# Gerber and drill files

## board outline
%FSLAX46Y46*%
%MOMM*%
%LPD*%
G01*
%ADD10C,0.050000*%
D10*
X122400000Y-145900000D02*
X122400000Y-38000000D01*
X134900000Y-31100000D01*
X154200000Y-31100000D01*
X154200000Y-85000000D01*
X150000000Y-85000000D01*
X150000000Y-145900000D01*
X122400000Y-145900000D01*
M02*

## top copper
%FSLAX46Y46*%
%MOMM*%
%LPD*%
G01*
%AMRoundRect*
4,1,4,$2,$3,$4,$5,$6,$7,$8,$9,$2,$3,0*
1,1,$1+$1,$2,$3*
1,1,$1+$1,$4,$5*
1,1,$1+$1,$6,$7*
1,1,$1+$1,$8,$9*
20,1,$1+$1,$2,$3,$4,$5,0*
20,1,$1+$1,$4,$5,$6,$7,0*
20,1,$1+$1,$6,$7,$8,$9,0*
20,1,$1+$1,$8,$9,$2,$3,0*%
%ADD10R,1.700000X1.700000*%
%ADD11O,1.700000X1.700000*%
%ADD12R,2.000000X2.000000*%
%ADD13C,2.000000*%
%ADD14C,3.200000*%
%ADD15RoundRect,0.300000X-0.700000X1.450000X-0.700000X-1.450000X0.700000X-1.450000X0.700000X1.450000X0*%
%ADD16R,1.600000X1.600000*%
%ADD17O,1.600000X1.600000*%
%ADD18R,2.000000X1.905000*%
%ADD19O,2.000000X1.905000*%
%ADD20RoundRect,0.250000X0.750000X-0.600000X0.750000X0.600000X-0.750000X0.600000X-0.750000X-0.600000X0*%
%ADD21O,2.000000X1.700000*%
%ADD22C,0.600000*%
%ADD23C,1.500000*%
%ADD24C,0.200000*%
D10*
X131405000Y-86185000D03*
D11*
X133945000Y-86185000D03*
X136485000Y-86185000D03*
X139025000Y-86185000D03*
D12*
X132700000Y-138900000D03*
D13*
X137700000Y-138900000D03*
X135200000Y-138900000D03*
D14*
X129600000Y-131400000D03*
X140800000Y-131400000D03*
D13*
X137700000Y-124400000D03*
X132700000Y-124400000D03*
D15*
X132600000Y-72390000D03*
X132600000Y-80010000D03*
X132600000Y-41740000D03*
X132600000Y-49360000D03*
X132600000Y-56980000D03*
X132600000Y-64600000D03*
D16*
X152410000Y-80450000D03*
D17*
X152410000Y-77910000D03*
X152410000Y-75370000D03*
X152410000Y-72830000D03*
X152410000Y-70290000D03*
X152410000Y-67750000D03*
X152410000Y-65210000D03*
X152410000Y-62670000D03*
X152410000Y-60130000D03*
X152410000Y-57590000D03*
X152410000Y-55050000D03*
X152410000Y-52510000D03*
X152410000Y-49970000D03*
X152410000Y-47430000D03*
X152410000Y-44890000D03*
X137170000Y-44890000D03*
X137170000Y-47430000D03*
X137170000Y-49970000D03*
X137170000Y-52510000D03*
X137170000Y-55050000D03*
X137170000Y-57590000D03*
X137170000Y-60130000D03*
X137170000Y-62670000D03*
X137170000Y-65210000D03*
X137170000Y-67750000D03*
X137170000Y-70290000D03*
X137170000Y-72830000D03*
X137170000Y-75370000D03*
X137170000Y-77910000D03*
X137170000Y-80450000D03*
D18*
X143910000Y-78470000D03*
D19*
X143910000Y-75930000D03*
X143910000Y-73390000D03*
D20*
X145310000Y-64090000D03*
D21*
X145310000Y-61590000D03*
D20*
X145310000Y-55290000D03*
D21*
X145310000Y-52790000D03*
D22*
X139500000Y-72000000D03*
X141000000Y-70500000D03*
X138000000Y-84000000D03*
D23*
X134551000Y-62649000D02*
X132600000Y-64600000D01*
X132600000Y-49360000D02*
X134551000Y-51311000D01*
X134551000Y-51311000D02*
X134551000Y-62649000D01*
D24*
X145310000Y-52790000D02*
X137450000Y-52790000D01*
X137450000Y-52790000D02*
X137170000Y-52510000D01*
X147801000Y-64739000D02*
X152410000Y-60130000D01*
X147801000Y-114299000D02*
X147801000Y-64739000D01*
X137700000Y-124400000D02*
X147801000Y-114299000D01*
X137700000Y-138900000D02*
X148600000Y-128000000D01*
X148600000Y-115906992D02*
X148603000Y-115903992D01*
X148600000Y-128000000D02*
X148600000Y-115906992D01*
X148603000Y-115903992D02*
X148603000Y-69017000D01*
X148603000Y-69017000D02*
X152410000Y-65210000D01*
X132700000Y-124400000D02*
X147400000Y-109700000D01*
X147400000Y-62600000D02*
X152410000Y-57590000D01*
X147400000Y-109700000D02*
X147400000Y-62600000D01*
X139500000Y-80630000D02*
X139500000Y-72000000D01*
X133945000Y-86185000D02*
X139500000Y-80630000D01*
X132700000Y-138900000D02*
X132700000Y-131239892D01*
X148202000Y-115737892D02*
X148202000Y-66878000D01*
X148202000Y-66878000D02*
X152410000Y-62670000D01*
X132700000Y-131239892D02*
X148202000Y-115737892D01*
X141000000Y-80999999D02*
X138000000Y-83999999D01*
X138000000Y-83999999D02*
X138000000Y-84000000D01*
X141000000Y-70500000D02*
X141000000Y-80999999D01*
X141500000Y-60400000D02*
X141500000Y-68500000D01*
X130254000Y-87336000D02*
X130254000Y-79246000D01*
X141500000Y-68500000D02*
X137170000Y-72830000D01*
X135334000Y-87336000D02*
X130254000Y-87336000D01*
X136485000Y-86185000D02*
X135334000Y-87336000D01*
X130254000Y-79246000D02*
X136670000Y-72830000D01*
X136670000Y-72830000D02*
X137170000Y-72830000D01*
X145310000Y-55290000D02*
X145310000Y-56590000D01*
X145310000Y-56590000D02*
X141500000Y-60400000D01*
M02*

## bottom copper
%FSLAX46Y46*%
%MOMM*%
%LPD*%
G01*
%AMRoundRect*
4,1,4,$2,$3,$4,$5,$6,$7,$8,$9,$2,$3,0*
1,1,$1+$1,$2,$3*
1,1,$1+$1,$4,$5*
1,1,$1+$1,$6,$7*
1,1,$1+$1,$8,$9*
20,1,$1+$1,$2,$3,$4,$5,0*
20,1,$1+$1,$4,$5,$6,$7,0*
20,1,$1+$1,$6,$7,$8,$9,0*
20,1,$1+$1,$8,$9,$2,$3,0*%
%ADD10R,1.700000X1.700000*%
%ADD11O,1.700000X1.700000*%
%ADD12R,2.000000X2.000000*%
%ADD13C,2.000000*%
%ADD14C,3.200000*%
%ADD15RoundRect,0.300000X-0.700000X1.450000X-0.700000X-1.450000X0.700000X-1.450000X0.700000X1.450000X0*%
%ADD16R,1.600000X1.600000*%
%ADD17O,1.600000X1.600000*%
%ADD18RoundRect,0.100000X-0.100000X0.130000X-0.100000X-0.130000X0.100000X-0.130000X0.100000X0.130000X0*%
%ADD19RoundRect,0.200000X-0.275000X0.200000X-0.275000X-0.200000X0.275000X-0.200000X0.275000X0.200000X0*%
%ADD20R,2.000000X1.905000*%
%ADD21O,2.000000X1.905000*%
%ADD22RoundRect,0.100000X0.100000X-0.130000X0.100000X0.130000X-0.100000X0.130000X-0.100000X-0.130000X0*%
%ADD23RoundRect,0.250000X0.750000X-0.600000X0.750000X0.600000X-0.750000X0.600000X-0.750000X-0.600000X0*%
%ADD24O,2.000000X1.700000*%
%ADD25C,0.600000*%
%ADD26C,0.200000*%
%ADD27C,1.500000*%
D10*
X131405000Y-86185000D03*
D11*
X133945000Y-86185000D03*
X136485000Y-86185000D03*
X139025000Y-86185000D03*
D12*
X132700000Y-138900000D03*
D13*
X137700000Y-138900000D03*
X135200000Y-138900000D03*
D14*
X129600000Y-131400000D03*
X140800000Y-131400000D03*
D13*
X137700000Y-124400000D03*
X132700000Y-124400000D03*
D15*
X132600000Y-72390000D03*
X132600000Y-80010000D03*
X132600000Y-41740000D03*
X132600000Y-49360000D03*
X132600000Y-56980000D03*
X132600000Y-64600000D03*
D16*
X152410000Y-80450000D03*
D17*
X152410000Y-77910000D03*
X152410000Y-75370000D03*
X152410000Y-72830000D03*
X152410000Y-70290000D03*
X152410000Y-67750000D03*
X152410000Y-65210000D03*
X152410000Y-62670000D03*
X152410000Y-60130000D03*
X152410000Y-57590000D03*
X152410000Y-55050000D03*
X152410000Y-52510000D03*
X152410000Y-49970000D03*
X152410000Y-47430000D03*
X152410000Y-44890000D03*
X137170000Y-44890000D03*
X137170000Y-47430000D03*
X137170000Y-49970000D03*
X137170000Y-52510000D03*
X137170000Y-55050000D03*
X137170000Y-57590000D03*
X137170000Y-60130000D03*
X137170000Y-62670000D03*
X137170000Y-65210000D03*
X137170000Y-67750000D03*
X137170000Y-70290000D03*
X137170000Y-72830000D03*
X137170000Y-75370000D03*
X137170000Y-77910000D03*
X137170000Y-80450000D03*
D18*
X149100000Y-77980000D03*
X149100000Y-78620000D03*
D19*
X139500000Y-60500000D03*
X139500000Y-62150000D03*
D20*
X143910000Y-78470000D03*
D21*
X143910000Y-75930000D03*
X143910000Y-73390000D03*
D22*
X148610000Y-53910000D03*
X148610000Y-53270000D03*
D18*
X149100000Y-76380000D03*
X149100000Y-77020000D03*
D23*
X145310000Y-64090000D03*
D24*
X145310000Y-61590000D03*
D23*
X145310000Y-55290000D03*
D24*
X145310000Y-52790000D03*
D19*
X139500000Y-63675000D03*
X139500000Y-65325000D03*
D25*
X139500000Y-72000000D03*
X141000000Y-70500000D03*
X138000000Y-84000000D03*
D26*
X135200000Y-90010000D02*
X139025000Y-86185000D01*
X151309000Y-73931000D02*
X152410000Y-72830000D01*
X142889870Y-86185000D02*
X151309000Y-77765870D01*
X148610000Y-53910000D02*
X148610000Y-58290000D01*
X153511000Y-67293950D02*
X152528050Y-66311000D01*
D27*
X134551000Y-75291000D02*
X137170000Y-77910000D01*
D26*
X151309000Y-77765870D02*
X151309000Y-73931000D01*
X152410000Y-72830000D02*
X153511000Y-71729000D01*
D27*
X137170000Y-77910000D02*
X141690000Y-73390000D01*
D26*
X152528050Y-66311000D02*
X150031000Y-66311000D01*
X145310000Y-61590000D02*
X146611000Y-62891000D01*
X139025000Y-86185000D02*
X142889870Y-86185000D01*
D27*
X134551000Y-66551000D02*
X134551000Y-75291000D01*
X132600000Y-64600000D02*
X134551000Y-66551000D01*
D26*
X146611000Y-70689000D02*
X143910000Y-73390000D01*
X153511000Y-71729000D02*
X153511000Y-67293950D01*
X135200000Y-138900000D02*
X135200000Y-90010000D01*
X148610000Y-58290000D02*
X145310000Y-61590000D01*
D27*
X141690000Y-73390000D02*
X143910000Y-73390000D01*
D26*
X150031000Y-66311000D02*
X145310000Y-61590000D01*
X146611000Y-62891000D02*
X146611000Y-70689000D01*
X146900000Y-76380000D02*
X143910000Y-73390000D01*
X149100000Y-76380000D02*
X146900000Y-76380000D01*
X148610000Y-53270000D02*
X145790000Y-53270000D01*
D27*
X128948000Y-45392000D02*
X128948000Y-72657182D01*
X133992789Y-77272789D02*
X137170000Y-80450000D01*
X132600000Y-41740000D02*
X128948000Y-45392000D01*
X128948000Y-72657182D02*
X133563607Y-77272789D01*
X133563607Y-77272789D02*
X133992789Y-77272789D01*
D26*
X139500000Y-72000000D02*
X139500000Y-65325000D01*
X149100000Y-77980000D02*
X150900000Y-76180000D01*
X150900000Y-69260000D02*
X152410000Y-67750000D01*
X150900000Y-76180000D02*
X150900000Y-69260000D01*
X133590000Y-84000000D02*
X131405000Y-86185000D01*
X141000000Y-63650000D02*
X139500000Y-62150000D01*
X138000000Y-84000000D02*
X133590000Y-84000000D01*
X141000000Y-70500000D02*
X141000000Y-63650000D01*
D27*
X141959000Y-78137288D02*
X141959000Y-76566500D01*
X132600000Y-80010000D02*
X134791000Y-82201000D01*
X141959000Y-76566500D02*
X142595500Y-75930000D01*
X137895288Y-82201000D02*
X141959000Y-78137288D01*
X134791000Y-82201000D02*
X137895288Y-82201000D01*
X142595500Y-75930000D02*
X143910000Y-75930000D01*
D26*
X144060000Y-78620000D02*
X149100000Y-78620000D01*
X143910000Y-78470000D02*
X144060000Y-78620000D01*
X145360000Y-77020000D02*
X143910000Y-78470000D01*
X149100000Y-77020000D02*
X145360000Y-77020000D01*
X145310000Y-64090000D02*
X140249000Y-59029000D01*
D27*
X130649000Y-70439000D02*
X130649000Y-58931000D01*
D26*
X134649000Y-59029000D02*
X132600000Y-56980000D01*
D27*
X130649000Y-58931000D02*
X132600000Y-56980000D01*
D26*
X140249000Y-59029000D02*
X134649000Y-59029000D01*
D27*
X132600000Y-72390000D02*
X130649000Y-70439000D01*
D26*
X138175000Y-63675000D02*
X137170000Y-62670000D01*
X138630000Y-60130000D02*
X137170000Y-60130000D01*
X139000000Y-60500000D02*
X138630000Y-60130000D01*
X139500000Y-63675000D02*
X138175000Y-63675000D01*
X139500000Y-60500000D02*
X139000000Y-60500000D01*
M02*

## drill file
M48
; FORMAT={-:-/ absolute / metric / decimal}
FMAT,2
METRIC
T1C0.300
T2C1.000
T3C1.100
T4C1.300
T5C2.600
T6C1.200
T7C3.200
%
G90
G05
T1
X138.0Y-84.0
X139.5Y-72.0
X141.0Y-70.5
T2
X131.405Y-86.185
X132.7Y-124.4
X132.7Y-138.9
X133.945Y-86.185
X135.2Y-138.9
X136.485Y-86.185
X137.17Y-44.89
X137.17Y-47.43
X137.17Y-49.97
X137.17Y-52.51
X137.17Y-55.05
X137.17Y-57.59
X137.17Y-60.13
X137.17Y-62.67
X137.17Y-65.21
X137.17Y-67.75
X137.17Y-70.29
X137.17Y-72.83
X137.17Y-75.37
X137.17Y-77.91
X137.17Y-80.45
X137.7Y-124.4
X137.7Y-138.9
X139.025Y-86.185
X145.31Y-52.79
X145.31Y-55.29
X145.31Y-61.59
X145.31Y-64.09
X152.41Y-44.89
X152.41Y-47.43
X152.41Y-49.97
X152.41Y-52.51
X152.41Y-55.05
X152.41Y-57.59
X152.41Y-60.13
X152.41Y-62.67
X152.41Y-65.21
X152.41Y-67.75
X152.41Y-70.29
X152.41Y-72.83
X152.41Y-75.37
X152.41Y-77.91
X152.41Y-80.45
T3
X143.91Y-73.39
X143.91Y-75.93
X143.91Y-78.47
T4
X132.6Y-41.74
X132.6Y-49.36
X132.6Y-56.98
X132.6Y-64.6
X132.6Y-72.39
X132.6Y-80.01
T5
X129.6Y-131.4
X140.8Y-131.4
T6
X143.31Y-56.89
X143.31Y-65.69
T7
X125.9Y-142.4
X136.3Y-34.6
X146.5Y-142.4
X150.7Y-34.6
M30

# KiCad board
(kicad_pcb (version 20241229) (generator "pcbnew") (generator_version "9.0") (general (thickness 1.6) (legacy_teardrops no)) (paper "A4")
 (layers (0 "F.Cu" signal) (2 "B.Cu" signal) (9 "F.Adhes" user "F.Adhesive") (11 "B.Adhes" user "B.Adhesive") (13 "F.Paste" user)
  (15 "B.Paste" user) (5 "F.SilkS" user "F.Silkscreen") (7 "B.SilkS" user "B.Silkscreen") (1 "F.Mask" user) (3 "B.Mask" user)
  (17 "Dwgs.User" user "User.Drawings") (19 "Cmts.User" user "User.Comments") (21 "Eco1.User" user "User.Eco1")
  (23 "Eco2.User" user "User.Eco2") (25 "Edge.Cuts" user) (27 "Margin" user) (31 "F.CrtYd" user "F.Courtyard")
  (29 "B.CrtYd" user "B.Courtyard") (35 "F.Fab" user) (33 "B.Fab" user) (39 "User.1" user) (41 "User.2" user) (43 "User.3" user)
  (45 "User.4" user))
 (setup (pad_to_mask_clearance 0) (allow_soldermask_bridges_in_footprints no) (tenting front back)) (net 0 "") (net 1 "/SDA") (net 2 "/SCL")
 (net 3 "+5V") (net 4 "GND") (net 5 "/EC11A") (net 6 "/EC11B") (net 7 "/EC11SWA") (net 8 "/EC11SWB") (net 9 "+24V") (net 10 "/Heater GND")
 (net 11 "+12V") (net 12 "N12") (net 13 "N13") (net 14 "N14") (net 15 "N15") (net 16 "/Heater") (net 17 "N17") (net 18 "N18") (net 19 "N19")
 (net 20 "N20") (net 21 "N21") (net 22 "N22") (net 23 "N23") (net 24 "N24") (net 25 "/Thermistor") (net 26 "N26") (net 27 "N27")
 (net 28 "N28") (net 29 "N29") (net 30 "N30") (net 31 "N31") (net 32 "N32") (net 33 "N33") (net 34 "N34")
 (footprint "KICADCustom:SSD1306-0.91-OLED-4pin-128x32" (layer "F.Cu") (at 129.215 122.685 90)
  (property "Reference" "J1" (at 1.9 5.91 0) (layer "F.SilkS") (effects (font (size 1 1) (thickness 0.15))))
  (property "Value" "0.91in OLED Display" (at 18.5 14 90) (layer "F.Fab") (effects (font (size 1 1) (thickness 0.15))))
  (pad "1" thru_hole rect (at 36.5 2.19 90) (size 1.7 1.7) (drill 1) (layers "*.Cu" "*.Mask") (remove_unused_layers no) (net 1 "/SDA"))
  (pad "2" thru_hole oval (at 36.5 4.73 90) (size 1.7 1.7) (drill 1) (layers "*.Cu" "*.Mask") (remove_unused_layers no) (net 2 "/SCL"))
  (pad "3" thru_hole oval (at 36.5 7.27 90) (size 1.7 1.7) (drill 1) (layers "*.Cu" "*.Mask") (remove_unused_layers no) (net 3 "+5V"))
  (pad "4" thru_hole oval (at 36.5 9.81 90) (size 1.7 1.7) (drill 1) (layers "*.Cu" "*.Mask") (remove_unused_layers no) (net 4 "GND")))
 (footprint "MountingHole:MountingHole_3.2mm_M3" (layer "F.Cu") (at 146.5 142.4)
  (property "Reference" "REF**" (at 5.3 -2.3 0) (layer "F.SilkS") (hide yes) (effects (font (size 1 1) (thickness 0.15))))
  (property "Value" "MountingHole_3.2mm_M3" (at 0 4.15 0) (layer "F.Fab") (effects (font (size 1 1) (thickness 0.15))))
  (pad "" np_thru_hole circle (at 0 0) (size 3.2 3.2) (drill 3.2) (layers "*.Cu" "*.Mask")))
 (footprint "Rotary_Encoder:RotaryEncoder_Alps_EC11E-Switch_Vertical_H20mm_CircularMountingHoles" (layer "F.Cu") (at 132.7 138.9 90)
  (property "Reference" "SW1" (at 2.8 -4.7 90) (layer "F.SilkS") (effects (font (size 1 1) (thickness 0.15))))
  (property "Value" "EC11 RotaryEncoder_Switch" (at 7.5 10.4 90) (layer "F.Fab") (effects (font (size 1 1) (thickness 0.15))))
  (pad "A" thru_hole rect (at 0 0 90) (size 2 2) (drill 1) (layers "*.Cu" "*.Mask") (remove_unused_layers no) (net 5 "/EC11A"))
  (pad "B" thru_hole circle (at 0 5 90) (size 2 2) (drill 1) (layers "*.Cu" "*.Mask") (remove_unused_layers no) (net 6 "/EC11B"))
  (pad "C" thru_hole circle (at 0 2.5 90) (size 2 2) (drill 1) (layers "*.Cu" "*.Mask") (remove_unused_layers no) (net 4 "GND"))
  (pad "MP" thru_hole circle (at 7.5 -3.1 90) (size 3.2 3.2) (drill 2.6) (layers "*.Cu" "*.Mask") (remove_unused_layers no))
  (pad "MP" thru_hole circle (at 7.5 8.1 90) (size 3.2 3.2) (drill 2.6) (layers "*.Cu" "*.Mask") (remove_unused_layers no))
  (pad "S1" thru_hole circle (at 14.5 5 90) (size 2 2) (drill 1) (layers "*.Cu" "*.Mask") (remove_unused_layers no) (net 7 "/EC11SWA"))
  (pad "S2" thru_hole circle (at 14.5 0 90) (size 2 2) (drill 1) (layers "*.Cu" "*.Mask") (remove_unused_layers no) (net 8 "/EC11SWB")))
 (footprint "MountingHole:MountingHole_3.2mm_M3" (layer "F.Cu") (at 136.3 34.6)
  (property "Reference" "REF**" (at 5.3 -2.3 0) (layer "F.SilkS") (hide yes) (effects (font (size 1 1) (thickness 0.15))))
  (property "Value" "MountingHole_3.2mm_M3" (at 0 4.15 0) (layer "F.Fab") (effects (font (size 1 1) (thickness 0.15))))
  (pad "" np_thru_hole circle (at 0 0) (size 3.2 3.2) (drill 3.2) (layers "*.Cu" "*.Mask")))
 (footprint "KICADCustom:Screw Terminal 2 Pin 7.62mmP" (layer "F.Cu") (at 132.6 72.39 -90)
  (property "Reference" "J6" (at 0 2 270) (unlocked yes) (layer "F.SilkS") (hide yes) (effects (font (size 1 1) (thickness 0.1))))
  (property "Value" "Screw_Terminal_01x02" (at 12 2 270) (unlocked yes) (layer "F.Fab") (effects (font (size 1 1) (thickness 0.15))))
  (pad "1" thru_hole roundrect (at 0 0 270) (size 3.5 2) (drill 1.3) (layers "*.Cu" "*.Mask") (remove_unused_layers no)
   (roundrect_rratio 0.15) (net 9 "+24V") (thermal_bridge_angle 45))
  (pad "2" thru_hole roundrect (at 7.62 0 270) (size 3.5 2) (drill 1.3) (layers "*.Cu" "*.Mask") (remove_unused_layers no)
   (roundrect_rratio 0.15) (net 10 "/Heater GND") (thermal_bridge_angle 45)))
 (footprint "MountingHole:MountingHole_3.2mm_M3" (layer "F.Cu") (at 150.7 34.6)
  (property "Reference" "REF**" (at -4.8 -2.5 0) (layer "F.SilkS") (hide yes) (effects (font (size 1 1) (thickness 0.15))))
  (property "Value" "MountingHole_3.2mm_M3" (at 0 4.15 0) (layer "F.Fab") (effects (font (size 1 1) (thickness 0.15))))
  (pad "" np_thru_hole circle (at 0 0) (size 3.2 3.2) (drill 3.2) (layers "*.Cu" "*.Mask")))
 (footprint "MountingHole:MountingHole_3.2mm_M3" (layer "F.Cu") (at 125.9 142.4)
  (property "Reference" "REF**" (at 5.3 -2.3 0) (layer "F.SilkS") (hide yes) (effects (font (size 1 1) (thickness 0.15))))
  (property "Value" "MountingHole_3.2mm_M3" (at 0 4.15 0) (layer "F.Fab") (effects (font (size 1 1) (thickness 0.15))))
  (pad "" np_thru_hole circle (at 0 0) (size 3.2 3.2) (drill 3.2) (layers "*.Cu" "*.Mask")))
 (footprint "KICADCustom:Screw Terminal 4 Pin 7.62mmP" (layer "F.Cu") (at 132.6 41.74 -90)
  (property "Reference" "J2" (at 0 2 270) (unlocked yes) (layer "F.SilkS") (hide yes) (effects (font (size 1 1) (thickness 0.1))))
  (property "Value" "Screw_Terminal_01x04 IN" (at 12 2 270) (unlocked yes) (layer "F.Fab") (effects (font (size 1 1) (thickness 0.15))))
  (pad "1" thru_hole roundrect (at 0 0 270) (size 3.5 2) (drill 1.3) (layers "*.Cu" "*.Mask") (remove_unused_layers no)
   (roundrect_rratio 0.15) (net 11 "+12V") (thermal_bridge_angle 45))
  (pad "2" thru_hole roundrect (at 7.62 0 270) (size 3.5 2) (drill 1.3) (layers "*.Cu" "*.Mask") (remove_unused_layers no)
   (roundrect_rratio 0.15) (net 4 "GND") (thermal_bridge_angle 45))
  (pad "3" thru_hole roundrect (at 15.24 0 270) (size 3.5 2) (drill 1.3) (layers "*.Cu" "*.Mask") (remove_unused_layers no)
   (roundrect_rratio 0.15) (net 9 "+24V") (thermal_bridge_angle 45))
  (pad "4" thru_hole roundrect (at 22.86 0 270) (size 3.5 2) (drill 1.3) (layers "*.Cu" "*.Mask") (remove_unused_layers no)
   (roundrect_rratio 0.15) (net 4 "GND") (thermal_bridge_angle 45)))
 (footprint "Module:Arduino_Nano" (layer "F.Cu") (at 152.41 80.45 180)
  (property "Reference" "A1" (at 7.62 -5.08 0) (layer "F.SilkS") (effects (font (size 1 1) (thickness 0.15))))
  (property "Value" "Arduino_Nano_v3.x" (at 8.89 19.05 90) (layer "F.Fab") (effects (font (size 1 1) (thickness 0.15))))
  (pad "1" thru_hole rect (at 0 0 180) (size 1.6 1.6) (drill 1) (layers "*.Cu" "*.Mask") (remove_unused_layers no) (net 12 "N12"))
  (pad "2" thru_hole oval (at 0 2.54 180) (size 1.6 1.6) (drill 1) (layers "*.Cu" "*.Mask") (remove_unused_layers no) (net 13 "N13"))
  (pad "3" thru_hole oval (at 0 5.08 180) (size 1.6 1.6) (drill 1) (layers "*.Cu" "*.Mask") (remove_unused_layers no) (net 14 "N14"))
  (pad "4" thru_hole oval (at 0 7.62 180) (size 1.6 1.6) (drill 1) (layers "*.Cu" "*.Mask") (remove_unused_layers no) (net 4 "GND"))
  (pad "5" thru_hole oval (at 0 10.16 180) (size 1.6 1.6) (drill 1) (layers "*.Cu" "*.Mask") (remove_unused_layers no) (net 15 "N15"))
  (pad "6" thru_hole oval (at 0 12.7 180) (size 1.6 1.6) (drill 1) (layers "*.Cu" "*.Mask") (remove_unused_layers no) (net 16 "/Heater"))
  (pad "7" thru_hole oval (at 0 15.24 180) (size 1.6 1.6) (drill 1) (layers "*.Cu" "*.Mask") (remove_unused_layers no) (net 6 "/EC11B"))
  (pad "8" thru_hole oval (at 0 17.78 180) (size 1.6 1.6) (drill 1) (layers "*.Cu" "*.Mask") (remove_unused_layers no) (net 5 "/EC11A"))
  (pad "9" thru_hole oval (at 0 20.32 180) (size 1.6 1.6) (drill 1) (layers "*.Cu" "*.Mask") (remove_unused_layers no) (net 7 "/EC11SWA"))
  (pad "10" thru_hole oval (at 0 22.86 180) (size 1.6 1.6) (drill 1) (layers "*.Cu" "*.Mask") (remove_unused_layers no) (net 8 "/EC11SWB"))
  (pad "11" thru_hole oval (at 0 25.4 180) (size 1.6 1.6) (drill 1) (layers "*.Cu" "*.Mask") (remove_unused_layers no) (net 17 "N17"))
  (pad "12" thru_hole oval (at 0 27.94 180) (size 1.6 1.6) (drill 1) (layers "*.Cu" "*.Mask") (remove_unused_layers no) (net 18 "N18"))
  (pad "13" thru_hole oval (at 0 30.48 180) (size 1.6 1.6) (drill 1) (layers "*.Cu" "*.Mask") (remove_unused_layers no) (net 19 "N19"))
  (pad "14" thru_hole oval (at 0 33.02 180) (size 1.6 1.6) (drill 1) (layers "*.Cu" "*.Mask") (remove_unused_layers no) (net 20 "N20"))
  (pad "15" thru_hole oval (at 0 35.56 180) (size 1.6 1.6) (drill 1) (layers "*.Cu" "*.Mask") (remove_unused_layers no) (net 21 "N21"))
  (pad "16" thru_hole oval (at 15.24 35.56 180) (size 1.6 1.6) (drill 1) (layers "*.Cu" "*.Mask") (remove_unused_layers no) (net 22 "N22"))
  (pad "17" thru_hole oval (at 15.24 33.02 180) (size 1.6 1.6) (drill 1) (layers "*.Cu" "*.Mask") (remove_unused_layers no) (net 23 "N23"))
  (pad "18" thru_hole oval (at 15.24 30.48 180) (size 1.6 1.6) (drill 1) (layers "*.Cu" "*.Mask") (remove_unused_layers no) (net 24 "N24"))
  (pad "19" thru_hole oval (at 15.24 27.94 180) (size 1.6 1.6) (drill 1) (layers "*.Cu" "*.Mask") (remove_unused_layers no)
   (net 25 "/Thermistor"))
  (pad "20" thru_hole oval (at 15.24 25.4 180) (size 1.6 1.6) (drill 1) (layers "*.Cu" "*.Mask") (remove_unused_layers no) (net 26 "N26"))
  (pad "21" thru_hole oval (at 15.24 22.86 180) (size 1.6 1.6) (drill 1) (layers "*.Cu" "*.Mask") (remove_unused_layers no) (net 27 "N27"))
  (pad "22" thru_hole oval (at 15.24 20.32 180) (size 1.6 1.6) (drill 1) (layers "*.Cu" "*.Mask") (remove_unused_layers no) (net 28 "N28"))
  (pad "23" thru_hole oval (at 15.24 17.78 180) (size 1.6 1.6) (drill 1) (layers "*.Cu" "*.Mask") (remove_unused_layers no) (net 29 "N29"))
  (pad "24" thru_hole oval (at 15.24 15.24 180) (size 1.6 1.6) (drill 1) (layers "*.Cu" "*.Mask") (remove_unused_layers no) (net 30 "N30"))
  (pad "25" thru_hole oval (at 15.24 12.7 180) (size 1.6 1.6) (drill 1) (layers "*.Cu" "*.Mask") (remove_unused_layers no) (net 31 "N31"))
  (pad "26" thru_hole oval (at 15.24 10.16 180) (size 1.6 1.6) (drill 1) (layers "*.Cu" "*.Mask") (remove_unused_layers no) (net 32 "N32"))
  (pad "27" thru_hole oval (at 15.24 7.62 180) (size 1.6 1.6) (drill 1) (layers "*.Cu" "*.Mask") (remove_unused_layers no) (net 3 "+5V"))
  (pad "28" thru_hole oval (at 15.24 5.08 180) (size 1.6 1.6) (drill 1) (layers "*.Cu" "*.Mask") (remove_unused_layers no) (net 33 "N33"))
  (pad "29" thru_hole oval (at 15.24 2.54 180) (size 1.6 1.6) (drill 1) (layers "*.Cu" "*.Mask") (remove_unused_layers no) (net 4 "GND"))
  (pad "30" thru_hole oval (at 15.24 0 180) (size 1.6 1.6) (drill 1) (layers "*.Cu" "*.Mask") (remove_unused_layers no) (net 11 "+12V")))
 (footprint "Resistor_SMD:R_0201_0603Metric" (layer "B.Cu") (at 149.1 78.3 -90)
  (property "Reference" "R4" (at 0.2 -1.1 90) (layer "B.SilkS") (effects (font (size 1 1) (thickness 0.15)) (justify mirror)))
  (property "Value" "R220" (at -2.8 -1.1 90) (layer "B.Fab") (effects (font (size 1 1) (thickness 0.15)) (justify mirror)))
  (pad "" smd roundrect (at -0.345 0 270) (size 0.318 0.36) (layers "B.Paste") (roundrect_rratio 0.25))
  (pad "" smd roundrect (at 0.345 0 270) (size 0.318 0.36) (layers "B.Paste") (roundrect_rratio 0.25))
  (pad "1" smd roundrect (at -0.32 0 270) (size 0.46 0.4) (layers "B.Cu" "B.Mask") (roundrect_rratio 0.25) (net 16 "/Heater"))
  (pad "2" smd roundrect (at 0.32 0 270) (size 0.46 0.4) (layers "B.Cu" "B.Mask") (roundrect_rratio 0.25) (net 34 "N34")))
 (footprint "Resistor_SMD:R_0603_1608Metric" (layer "B.Cu") (at 139.5 61.325 -90)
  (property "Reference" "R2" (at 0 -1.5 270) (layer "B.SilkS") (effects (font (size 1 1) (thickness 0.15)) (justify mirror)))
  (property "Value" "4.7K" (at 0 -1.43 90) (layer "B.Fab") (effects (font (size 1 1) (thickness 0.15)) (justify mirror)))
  (pad "1" smd roundrect (at -0.825 0 270) (size 0.8 0.95) (layers "B.Cu" "B.Mask" "B.Paste") (roundrect_rratio 0.25) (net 29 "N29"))
  (pad "2" smd roundrect (at 0.825 0 270) (size 0.8 0.95) (layers "B.Cu" "B.Mask" "B.Paste") (roundrect_rratio 0.25) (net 1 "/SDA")))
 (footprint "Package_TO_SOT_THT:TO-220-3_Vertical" (layer "B.Cu") (at 143.91 78.47 90)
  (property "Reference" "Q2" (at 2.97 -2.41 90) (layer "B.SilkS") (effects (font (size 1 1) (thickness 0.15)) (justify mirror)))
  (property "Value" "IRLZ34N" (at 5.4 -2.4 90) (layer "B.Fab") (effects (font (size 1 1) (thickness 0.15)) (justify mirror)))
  (pad "1" thru_hole rect (at 0 0 90) (size 1.905 2) (drill 1.1) (layers "*.Cu" "*.Mask") (remove_unused_layers no) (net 34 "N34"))
  (pad "2" thru_hole oval (at 2.54 0 90) (size 1.905 2) (drill 1.1) (layers "*.Cu" "*.Mask") (remove_unused_layers no)
   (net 10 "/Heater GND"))
  (pad "3" thru_hole oval (at 5.08 0 90) (size 1.905 2) (drill 1.1) (layers "*.Cu" "*.Mask") (remove_unused_layers no) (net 4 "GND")))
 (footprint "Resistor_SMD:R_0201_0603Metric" (layer "B.Cu") (at 148.61 53.59 90)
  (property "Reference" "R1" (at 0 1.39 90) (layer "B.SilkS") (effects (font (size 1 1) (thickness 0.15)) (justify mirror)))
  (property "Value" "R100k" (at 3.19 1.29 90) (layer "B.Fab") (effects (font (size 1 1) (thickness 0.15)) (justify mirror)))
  (pad "" smd roundrect (at -0.345 0 90) (size 0.318 0.36) (layers "B.Paste") (roundrect_rratio 0.25))
  (pad "" smd roundrect (at 0.345 0 90) (size 0.318 0.36) (layers "B.Paste") (roundrect_rratio 0.25))
  (pad "1" smd roundrect (at -0.32 0 90) (size 0.46 0.4) (layers "B.Cu" "B.Mask") (roundrect_rratio 0.25) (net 4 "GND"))
  (pad "2" smd roundrect (at 0.32 0 90) (size 0.46 0.4) (layers "B.Cu" "B.Mask") (roundrect_rratio 0.25) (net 25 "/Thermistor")))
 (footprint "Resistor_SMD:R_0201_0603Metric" (layer "B.Cu") (at 149.1 76.7 -90)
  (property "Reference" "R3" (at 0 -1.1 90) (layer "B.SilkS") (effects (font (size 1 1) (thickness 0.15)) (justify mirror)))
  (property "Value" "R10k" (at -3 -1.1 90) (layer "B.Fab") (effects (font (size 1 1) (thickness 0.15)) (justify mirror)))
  (pad "" smd roundrect (at -0.345 0 270) (size 0.318 0.36) (layers "B.Paste") (roundrect_rratio 0.25))
  (pad "" smd roundrect (at 0.345 0 270) (size 0.318 0.36) (layers "B.Paste") (roundrect_rratio 0.25))
  (pad "1" smd roundrect (at -0.32 0 270) (size 0.46 0.4) (layers "B.Cu" "B.Mask") (roundrect_rratio 0.25) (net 4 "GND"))
  (pad "2" smd roundrect (at 0.32 0 270) (size 0.46 0.4) (layers "B.Cu" "B.Mask") (roundrect_rratio 0.25) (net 34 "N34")))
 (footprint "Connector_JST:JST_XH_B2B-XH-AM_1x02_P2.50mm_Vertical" (layer "B.Cu") (at 145.31 64.09 90)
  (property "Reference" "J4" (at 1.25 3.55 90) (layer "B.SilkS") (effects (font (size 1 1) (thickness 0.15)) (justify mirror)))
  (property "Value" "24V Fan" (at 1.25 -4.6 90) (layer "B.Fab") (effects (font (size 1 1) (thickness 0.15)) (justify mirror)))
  (pad "" np_thru_hole circle (at -1.6 -2 90) (size 1.2 1.2) (drill 1.2) (layers "*.Cu" "*.Mask"))
  (pad "1" thru_hole roundrect (at 0 0 90) (size 1.7 2) (drill 1) (layers "*.Cu" "*.Mask") (remove_unused_layers no)
   (roundrect_rratio 0.147059) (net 9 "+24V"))
  (pad "2" thru_hole oval (at 2.5 0 90) (size 1.7 2) (drill 1) (layers "*.Cu" "*.Mask") (remove_unused_layers no) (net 4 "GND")))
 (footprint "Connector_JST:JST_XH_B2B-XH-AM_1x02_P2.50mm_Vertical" (layer "B.Cu") (at 145.31 55.29 90)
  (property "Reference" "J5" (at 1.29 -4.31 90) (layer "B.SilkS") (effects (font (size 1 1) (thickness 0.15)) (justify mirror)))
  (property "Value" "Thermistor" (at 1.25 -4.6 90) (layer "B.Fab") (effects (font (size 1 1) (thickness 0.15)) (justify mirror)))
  (pad "" np_thru_hole circle (at -1.6 -2 90) (size 1.2 1.2) (drill 1.2) (layers "*.Cu" "*.Mask"))
  (pad "1" thru_hole roundrect (at 0 0 90) (size 1.7 2) (drill 1) (layers "*.Cu" "*.Mask") (remove_unused_layers no)
   (roundrect_rratio 0.147059) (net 3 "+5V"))
  (pad "2" thru_hole oval (at 2.5 0 90) (size 1.7 2) (drill 1) (layers "*.Cu" "*.Mask") (remove_unused_layers no) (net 25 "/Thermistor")))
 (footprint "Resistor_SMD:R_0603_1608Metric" (layer "B.Cu") (at 139.5 64.5 -90)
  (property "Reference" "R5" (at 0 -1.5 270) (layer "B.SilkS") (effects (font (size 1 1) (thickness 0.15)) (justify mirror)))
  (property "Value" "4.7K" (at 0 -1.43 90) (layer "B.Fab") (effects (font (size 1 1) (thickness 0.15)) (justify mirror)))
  (pad "1" smd roundrect (at -0.825 0 270) (size 0.8 0.95) (layers "B.Cu" "B.Mask" "B.Paste") (roundrect_rratio 0.25) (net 30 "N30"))
  (pad "2" smd roundrect (at 0.825 0 270) (size 0.8 0.95) (layers "B.Cu" "B.Mask" "B.Paste") (roundrect_rratio 0.25) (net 2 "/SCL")))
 (gr_poly
  (pts (xy 122.4 145.9) (xy 122.4 38) (xy 134.9 31.1) (xy 154.2 31.1) (xy 154.2 85) (xy 150 85) (xy 150 145.9))
  (stroke (width 0.05) (type solid)) (fill no) (layer "Edge.Cuts"))
 (segment (start 134.551 62.649) (end 132.6 64.6) (width 1.5) (layer "F.Cu") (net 4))
 (segment (start 132.6 49.36) (end 134.551 51.311) (width 1.5) (layer "F.Cu") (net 4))
 (segment (start 134.551 51.311) (end 134.551 62.649) (width 1.5) (layer "F.Cu") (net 4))
 (segment (start 135.2 90.01) (end 139.025 86.185) (width 0.2) (layer "B.Cu") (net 4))
 (segment (start 151.309 73.931) (end 152.41 72.83) (width 0.2) (layer "B.Cu") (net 4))
 (segment (start 142.88987 86.185) (end 151.309 77.76587) (width 0.2) (layer "B.Cu") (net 4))
 (segment (start 148.61 53.91) (end 148.61 58.29) (width 0.2) (layer "B.Cu") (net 4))
 (segment (start 153.511 67.29395) (end 152.52805 66.311) (width 0.2) (layer "B.Cu") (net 4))
 (segment (start 134.551 75.291) (end 137.17 77.91) (width 1.5) (layer "B.Cu") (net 4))
 (segment (start 151.309 77.76587) (end 151.309 73.931) (width 0.2) (layer "B.Cu") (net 4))
 (segment (start 152.41 72.83) (end 153.511 71.729) (width 0.2) (layer "B.Cu") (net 4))
 (segment (start 137.17 77.91) (end 141.69 73.39) (width 1.5) (layer "B.Cu") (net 4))
 (segment (start 152.52805 66.311) (end 150.031 66.311) (width 0.2) (layer "B.Cu") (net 4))
 (segment (start 145.31 61.59) (end 146.611 62.891) (width 0.2) (layer "B.Cu") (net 4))
 (segment (start 139.025 86.185) (end 142.88987 86.185) (width 0.2) (layer "B.Cu") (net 4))
 (segment (start 134.551 66.551) (end 134.551 75.291) (width 1.5) (layer "B.Cu") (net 4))
 (segment (start 132.6 64.6) (end 134.551 66.551) (width 1.5) (layer "B.Cu") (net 4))
 (segment (start 146.611 70.689) (end 143.91 73.39) (width 0.2) (layer "B.Cu") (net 4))
 (segment (start 153.511 71.729) (end 153.511 67.29395) (width 0.2) (layer "B.Cu") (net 4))
 (segment (start 135.2 138.9) (end 135.2 90.01) (width 0.2) (layer "B.Cu") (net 4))
 (segment (start 148.61 58.29) (end 145.31 61.59) (width 0.2) (layer "B.Cu") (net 4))
 (segment (start 141.69 73.39) (end 143.91 73.39) (width 1.5) (layer "B.Cu") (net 4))
 (segment (start 150.031 66.311) (end 145.31 61.59) (width 0.2) (layer "B.Cu") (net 4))
 (segment (start 146.611 62.891) (end 146.611 70.689) (width 0.2) (layer "B.Cu") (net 4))
 (segment (start 146.9 76.38) (end 143.91 73.39) (width 0.2) (layer "B.Cu") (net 4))
 (segment (start 149.1 76.38) (end 146.9 76.38) (width 0.2) (layer "B.Cu") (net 4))
 (segment (start 145.31 52.79) (end 137.45 52.79) (width 0.2) (layer "F.Cu") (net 25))
 (segment (start 137.45 52.79) (end 137.17 52.51) (width 0.2) (layer "F.Cu") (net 25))
 (segment (start 148.61 53.27) (end 145.79 53.27) (width 0.2) (layer "B.Cu") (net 25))
 (segment (start 147.801 64.739) (end 152.41 60.13) (width 0.2) (layer "F.Cu") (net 7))
 (segment (start 147.801 114.299) (end 147.801 64.739) (width 0.2) (layer "F.Cu") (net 7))
 (segment (start 137.7 124.4) (end 147.801 114.299) (width 0.2) (layer "F.Cu") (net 7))
 (segment (start 137.7 138.9) (end 148.6 128) (width 0.2) (layer "F.Cu") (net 6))
 (segment (start 148.6 115.906992) (end 148.603 115.903992) (width 0.2) (layer "F.Cu") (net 6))
 (segment (start 148.6 128) (end 148.6 115.906992) (width 0.2) (layer "F.Cu") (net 6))
 (segment (start 148.603 115.903992) (end 148.603 69.017) (width 0.2) (layer "F.Cu") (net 6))
 (segment (start 148.603 69.017) (end 152.41 65.21) (width 0.2) (layer "F.Cu") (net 6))
 (segment (start 132.7 124.4) (end 147.4 109.7) (width 0.2) (layer "F.Cu") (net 8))
 (segment (start 147.4 62.6) (end 152.41 57.59) (width 0.2) (layer "F.Cu") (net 8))
 (segment (start 147.4 109.7) (end 147.4 62.6) (width 0.2) (layer "F.Cu") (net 8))
 (segment (start 128.948 45.392) (end 128.948 72.657182) (width 1.5) (layer "B.Cu") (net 11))
 (segment (start 133.992789 77.272789) (end 137.17 80.45) (width 1.5) (layer "B.Cu") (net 11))
 (segment (start 132.6 41.74) (end 128.948 45.392) (width 1.5) (layer "B.Cu") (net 11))
 (segment (start 128.948 72.657182) (end 133.563607 77.272789) (width 1.5) (layer "B.Cu") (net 11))
 (segment (start 133.563607 77.272789) (end 133.992789 77.272789) (width 1.5) (layer "B.Cu") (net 11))
 (segment (start 139.5 80.63) (end 139.5 72) (width 0.2) (layer "F.Cu") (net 2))
 (segment (start 133.945 86.185) (end 139.5 80.63) (width 0.2) (layer "F.Cu") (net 2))
 (via (at 139.5 72) (size 0.6) (drill 0.3) (layers "F.Cu" "B.Cu") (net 2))
 (segment (start 139.5 72) (end 139.5 65.325) (width 0.2) (layer "B.Cu") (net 2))
 (segment (start 132.7 138.9) (end 132.7 131.239892) (width 0.2) (layer "F.Cu") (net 5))
 (segment (start 148.202 115.737892) (end 148.202 66.878) (width 0.2) (layer "F.Cu") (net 5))
 (segment (start 148.202 66.878) (end 152.41 62.67) (width 0.2) (layer "F.Cu") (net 5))
 (segment (start 132.7 131.239892) (end 148.202 115.737892) (width 0.2) (layer "F.Cu") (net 5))
 (segment (start 149.1 77.98) (end 150.9 76.18) (width 0.2) (layer "B.Cu") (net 16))
 (segment (start 150.9 69.26) (end 152.41 67.75) (width 0.2) (layer "B.Cu") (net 16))
 (segment (start 150.9 76.18) (end 150.9 69.26) (width 0.2) (layer "B.Cu") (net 16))
 (segment (start 141 80.999999) (end 138 83.999999) (width 0.2) (layer "F.Cu") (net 1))
 (segment (start 138 83.999999) (end 138 84) (width 0.2) (layer "F.Cu") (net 1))
 (segment (start 141 70.5) (end 141 80.999999) (width 0.2) (layer "F.Cu") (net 1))
 (via (at 141 70.5) (size 0.6) (drill 0.3) (layers "F.Cu" "B.Cu") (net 1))
 (via (at 138 84) (size 0.6) (drill 0.3) (layers "F.Cu" "B.Cu") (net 1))
 (segment (start 133.59 84) (end 131.405 86.185) (width 0.2) (layer "B.Cu") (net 1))
 (segment (start 141 63.65) (end 139.5 62.15) (width 0.2) (layer "B.Cu") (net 1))
 (segment (start 138 84) (end 133.59 84) (width 0.2) (layer "B.Cu") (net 1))
 (segment (start 141 70.5) (end 141 63.65) (width 0.2) (layer "B.Cu") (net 1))
 (segment (start 141.5 60.4) (end 141.5 68.5) (width 0.2) (layer "F.Cu") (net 3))
 (segment (start 130.254 87.336) (end 130.254 79.246) (width 0.2) (layer "F.Cu") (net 3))
 (segment (start 141.5 68.5) (end 137.17 72.83) (width 0.2) (layer "F.Cu") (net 3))
 (segment (start 135.334 87.336) (end 130.254 87.336) (width 0.2) (layer "F.Cu") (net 3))
 (segment (start 136.485 86.185) (end 135.334 87.336) (width 0.2) (layer "F.Cu") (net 3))
 (segment (start 130.254 79.246) (end 136.67 72.83) (width 0.2) (layer "F.Cu") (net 3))
 (segment (start 136.67 72.83) (end 137.17 72.83) (width 0.2) (layer "F.Cu") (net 3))
 (segment (start 145.31 55.29) (end 145.31 56.59) (width 0.2) (layer "F.Cu") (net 3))
 (segment (start 145.31 56.59) (end 141.5 60.4) (width 0.2) (layer "F.Cu") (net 3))
 (segment (start 141.959 78.137288) (end 141.959 76.5665) (width 1.5) (layer "B.Cu") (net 10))
 (segment (start 132.6 80.01) (end 134.791 82.201) (width 1.5) (layer "B.Cu") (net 10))
 (segment (start 141.959 76.5665) (end 142.5955 75.93) (width 1.5) (layer "B.Cu") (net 10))
 (segment (start 137.895288 82.201) (end 141.959 78.137288) (width 1.5) (layer "B.Cu") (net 10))
 (segment (start 134.791 82.201) (end 137.895288 82.201) (width 1.5) (layer "B.Cu") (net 10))
 (segment (start 142.5955 75.93) (end 143.91 75.93) (width 1.5) (layer "B.Cu") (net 10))
 (segment (start 144.06 78.62) (end 149.1 78.62) (width 0.2) (layer "B.Cu") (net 34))
 (segment (start 143.91 78.47) (end 144.06 78.62) (width 0.2) (layer "B.Cu") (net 34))
 (segment (start 145.36 77.02) (end 143.91 78.47) (width 0.2) (layer "B.Cu") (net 34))
 (segment (start 149.1 77.02) (end 145.36 77.02) (width 0.2) (layer "B.Cu") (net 34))
 (segment (start 145.31 64.09) (end 140.249 59.029) (width 0.2) (layer "B.Cu") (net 9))
 (segment (start 130.649 70.439) (end 130.649 58.931) (width 1.5) (layer "B.Cu") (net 9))
 (segment (start 134.649 59.029) (end 132.6 56.98) (width 0.2) (layer "B.Cu") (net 9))
 (segment (start 130.649 58.931) (end 132.6 56.98) (width 1.5) (layer "B.Cu") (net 9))
 (segment (start 140.249 59.029) (end 134.649 59.029) (width 0.2) (layer "B.Cu") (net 9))
 (segment (start 132.6 72.39) (end 130.649 70.439) (width 1.5) (layer "B.Cu") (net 9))
 (segment (start 138.175 63.675) (end 137.17 62.67) (width 0.2) (layer "B.Cu") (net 29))
 (segment (start 138.63 60.13) (end 137.17 60.13) (width 0.2) (layer "B.Cu") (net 29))
 (segment (start 139 60.5) (end 138.63 60.13) (width 0.2) (layer "B.Cu") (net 29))
 (segment (start 139.5 63.675) (end 138.175 63.675) (width 0.2) (layer "B.Cu") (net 29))
 (segment (start 139.5 60.5) (end 139 60.5) (width 0.2) (layer "B.Cu") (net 29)))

